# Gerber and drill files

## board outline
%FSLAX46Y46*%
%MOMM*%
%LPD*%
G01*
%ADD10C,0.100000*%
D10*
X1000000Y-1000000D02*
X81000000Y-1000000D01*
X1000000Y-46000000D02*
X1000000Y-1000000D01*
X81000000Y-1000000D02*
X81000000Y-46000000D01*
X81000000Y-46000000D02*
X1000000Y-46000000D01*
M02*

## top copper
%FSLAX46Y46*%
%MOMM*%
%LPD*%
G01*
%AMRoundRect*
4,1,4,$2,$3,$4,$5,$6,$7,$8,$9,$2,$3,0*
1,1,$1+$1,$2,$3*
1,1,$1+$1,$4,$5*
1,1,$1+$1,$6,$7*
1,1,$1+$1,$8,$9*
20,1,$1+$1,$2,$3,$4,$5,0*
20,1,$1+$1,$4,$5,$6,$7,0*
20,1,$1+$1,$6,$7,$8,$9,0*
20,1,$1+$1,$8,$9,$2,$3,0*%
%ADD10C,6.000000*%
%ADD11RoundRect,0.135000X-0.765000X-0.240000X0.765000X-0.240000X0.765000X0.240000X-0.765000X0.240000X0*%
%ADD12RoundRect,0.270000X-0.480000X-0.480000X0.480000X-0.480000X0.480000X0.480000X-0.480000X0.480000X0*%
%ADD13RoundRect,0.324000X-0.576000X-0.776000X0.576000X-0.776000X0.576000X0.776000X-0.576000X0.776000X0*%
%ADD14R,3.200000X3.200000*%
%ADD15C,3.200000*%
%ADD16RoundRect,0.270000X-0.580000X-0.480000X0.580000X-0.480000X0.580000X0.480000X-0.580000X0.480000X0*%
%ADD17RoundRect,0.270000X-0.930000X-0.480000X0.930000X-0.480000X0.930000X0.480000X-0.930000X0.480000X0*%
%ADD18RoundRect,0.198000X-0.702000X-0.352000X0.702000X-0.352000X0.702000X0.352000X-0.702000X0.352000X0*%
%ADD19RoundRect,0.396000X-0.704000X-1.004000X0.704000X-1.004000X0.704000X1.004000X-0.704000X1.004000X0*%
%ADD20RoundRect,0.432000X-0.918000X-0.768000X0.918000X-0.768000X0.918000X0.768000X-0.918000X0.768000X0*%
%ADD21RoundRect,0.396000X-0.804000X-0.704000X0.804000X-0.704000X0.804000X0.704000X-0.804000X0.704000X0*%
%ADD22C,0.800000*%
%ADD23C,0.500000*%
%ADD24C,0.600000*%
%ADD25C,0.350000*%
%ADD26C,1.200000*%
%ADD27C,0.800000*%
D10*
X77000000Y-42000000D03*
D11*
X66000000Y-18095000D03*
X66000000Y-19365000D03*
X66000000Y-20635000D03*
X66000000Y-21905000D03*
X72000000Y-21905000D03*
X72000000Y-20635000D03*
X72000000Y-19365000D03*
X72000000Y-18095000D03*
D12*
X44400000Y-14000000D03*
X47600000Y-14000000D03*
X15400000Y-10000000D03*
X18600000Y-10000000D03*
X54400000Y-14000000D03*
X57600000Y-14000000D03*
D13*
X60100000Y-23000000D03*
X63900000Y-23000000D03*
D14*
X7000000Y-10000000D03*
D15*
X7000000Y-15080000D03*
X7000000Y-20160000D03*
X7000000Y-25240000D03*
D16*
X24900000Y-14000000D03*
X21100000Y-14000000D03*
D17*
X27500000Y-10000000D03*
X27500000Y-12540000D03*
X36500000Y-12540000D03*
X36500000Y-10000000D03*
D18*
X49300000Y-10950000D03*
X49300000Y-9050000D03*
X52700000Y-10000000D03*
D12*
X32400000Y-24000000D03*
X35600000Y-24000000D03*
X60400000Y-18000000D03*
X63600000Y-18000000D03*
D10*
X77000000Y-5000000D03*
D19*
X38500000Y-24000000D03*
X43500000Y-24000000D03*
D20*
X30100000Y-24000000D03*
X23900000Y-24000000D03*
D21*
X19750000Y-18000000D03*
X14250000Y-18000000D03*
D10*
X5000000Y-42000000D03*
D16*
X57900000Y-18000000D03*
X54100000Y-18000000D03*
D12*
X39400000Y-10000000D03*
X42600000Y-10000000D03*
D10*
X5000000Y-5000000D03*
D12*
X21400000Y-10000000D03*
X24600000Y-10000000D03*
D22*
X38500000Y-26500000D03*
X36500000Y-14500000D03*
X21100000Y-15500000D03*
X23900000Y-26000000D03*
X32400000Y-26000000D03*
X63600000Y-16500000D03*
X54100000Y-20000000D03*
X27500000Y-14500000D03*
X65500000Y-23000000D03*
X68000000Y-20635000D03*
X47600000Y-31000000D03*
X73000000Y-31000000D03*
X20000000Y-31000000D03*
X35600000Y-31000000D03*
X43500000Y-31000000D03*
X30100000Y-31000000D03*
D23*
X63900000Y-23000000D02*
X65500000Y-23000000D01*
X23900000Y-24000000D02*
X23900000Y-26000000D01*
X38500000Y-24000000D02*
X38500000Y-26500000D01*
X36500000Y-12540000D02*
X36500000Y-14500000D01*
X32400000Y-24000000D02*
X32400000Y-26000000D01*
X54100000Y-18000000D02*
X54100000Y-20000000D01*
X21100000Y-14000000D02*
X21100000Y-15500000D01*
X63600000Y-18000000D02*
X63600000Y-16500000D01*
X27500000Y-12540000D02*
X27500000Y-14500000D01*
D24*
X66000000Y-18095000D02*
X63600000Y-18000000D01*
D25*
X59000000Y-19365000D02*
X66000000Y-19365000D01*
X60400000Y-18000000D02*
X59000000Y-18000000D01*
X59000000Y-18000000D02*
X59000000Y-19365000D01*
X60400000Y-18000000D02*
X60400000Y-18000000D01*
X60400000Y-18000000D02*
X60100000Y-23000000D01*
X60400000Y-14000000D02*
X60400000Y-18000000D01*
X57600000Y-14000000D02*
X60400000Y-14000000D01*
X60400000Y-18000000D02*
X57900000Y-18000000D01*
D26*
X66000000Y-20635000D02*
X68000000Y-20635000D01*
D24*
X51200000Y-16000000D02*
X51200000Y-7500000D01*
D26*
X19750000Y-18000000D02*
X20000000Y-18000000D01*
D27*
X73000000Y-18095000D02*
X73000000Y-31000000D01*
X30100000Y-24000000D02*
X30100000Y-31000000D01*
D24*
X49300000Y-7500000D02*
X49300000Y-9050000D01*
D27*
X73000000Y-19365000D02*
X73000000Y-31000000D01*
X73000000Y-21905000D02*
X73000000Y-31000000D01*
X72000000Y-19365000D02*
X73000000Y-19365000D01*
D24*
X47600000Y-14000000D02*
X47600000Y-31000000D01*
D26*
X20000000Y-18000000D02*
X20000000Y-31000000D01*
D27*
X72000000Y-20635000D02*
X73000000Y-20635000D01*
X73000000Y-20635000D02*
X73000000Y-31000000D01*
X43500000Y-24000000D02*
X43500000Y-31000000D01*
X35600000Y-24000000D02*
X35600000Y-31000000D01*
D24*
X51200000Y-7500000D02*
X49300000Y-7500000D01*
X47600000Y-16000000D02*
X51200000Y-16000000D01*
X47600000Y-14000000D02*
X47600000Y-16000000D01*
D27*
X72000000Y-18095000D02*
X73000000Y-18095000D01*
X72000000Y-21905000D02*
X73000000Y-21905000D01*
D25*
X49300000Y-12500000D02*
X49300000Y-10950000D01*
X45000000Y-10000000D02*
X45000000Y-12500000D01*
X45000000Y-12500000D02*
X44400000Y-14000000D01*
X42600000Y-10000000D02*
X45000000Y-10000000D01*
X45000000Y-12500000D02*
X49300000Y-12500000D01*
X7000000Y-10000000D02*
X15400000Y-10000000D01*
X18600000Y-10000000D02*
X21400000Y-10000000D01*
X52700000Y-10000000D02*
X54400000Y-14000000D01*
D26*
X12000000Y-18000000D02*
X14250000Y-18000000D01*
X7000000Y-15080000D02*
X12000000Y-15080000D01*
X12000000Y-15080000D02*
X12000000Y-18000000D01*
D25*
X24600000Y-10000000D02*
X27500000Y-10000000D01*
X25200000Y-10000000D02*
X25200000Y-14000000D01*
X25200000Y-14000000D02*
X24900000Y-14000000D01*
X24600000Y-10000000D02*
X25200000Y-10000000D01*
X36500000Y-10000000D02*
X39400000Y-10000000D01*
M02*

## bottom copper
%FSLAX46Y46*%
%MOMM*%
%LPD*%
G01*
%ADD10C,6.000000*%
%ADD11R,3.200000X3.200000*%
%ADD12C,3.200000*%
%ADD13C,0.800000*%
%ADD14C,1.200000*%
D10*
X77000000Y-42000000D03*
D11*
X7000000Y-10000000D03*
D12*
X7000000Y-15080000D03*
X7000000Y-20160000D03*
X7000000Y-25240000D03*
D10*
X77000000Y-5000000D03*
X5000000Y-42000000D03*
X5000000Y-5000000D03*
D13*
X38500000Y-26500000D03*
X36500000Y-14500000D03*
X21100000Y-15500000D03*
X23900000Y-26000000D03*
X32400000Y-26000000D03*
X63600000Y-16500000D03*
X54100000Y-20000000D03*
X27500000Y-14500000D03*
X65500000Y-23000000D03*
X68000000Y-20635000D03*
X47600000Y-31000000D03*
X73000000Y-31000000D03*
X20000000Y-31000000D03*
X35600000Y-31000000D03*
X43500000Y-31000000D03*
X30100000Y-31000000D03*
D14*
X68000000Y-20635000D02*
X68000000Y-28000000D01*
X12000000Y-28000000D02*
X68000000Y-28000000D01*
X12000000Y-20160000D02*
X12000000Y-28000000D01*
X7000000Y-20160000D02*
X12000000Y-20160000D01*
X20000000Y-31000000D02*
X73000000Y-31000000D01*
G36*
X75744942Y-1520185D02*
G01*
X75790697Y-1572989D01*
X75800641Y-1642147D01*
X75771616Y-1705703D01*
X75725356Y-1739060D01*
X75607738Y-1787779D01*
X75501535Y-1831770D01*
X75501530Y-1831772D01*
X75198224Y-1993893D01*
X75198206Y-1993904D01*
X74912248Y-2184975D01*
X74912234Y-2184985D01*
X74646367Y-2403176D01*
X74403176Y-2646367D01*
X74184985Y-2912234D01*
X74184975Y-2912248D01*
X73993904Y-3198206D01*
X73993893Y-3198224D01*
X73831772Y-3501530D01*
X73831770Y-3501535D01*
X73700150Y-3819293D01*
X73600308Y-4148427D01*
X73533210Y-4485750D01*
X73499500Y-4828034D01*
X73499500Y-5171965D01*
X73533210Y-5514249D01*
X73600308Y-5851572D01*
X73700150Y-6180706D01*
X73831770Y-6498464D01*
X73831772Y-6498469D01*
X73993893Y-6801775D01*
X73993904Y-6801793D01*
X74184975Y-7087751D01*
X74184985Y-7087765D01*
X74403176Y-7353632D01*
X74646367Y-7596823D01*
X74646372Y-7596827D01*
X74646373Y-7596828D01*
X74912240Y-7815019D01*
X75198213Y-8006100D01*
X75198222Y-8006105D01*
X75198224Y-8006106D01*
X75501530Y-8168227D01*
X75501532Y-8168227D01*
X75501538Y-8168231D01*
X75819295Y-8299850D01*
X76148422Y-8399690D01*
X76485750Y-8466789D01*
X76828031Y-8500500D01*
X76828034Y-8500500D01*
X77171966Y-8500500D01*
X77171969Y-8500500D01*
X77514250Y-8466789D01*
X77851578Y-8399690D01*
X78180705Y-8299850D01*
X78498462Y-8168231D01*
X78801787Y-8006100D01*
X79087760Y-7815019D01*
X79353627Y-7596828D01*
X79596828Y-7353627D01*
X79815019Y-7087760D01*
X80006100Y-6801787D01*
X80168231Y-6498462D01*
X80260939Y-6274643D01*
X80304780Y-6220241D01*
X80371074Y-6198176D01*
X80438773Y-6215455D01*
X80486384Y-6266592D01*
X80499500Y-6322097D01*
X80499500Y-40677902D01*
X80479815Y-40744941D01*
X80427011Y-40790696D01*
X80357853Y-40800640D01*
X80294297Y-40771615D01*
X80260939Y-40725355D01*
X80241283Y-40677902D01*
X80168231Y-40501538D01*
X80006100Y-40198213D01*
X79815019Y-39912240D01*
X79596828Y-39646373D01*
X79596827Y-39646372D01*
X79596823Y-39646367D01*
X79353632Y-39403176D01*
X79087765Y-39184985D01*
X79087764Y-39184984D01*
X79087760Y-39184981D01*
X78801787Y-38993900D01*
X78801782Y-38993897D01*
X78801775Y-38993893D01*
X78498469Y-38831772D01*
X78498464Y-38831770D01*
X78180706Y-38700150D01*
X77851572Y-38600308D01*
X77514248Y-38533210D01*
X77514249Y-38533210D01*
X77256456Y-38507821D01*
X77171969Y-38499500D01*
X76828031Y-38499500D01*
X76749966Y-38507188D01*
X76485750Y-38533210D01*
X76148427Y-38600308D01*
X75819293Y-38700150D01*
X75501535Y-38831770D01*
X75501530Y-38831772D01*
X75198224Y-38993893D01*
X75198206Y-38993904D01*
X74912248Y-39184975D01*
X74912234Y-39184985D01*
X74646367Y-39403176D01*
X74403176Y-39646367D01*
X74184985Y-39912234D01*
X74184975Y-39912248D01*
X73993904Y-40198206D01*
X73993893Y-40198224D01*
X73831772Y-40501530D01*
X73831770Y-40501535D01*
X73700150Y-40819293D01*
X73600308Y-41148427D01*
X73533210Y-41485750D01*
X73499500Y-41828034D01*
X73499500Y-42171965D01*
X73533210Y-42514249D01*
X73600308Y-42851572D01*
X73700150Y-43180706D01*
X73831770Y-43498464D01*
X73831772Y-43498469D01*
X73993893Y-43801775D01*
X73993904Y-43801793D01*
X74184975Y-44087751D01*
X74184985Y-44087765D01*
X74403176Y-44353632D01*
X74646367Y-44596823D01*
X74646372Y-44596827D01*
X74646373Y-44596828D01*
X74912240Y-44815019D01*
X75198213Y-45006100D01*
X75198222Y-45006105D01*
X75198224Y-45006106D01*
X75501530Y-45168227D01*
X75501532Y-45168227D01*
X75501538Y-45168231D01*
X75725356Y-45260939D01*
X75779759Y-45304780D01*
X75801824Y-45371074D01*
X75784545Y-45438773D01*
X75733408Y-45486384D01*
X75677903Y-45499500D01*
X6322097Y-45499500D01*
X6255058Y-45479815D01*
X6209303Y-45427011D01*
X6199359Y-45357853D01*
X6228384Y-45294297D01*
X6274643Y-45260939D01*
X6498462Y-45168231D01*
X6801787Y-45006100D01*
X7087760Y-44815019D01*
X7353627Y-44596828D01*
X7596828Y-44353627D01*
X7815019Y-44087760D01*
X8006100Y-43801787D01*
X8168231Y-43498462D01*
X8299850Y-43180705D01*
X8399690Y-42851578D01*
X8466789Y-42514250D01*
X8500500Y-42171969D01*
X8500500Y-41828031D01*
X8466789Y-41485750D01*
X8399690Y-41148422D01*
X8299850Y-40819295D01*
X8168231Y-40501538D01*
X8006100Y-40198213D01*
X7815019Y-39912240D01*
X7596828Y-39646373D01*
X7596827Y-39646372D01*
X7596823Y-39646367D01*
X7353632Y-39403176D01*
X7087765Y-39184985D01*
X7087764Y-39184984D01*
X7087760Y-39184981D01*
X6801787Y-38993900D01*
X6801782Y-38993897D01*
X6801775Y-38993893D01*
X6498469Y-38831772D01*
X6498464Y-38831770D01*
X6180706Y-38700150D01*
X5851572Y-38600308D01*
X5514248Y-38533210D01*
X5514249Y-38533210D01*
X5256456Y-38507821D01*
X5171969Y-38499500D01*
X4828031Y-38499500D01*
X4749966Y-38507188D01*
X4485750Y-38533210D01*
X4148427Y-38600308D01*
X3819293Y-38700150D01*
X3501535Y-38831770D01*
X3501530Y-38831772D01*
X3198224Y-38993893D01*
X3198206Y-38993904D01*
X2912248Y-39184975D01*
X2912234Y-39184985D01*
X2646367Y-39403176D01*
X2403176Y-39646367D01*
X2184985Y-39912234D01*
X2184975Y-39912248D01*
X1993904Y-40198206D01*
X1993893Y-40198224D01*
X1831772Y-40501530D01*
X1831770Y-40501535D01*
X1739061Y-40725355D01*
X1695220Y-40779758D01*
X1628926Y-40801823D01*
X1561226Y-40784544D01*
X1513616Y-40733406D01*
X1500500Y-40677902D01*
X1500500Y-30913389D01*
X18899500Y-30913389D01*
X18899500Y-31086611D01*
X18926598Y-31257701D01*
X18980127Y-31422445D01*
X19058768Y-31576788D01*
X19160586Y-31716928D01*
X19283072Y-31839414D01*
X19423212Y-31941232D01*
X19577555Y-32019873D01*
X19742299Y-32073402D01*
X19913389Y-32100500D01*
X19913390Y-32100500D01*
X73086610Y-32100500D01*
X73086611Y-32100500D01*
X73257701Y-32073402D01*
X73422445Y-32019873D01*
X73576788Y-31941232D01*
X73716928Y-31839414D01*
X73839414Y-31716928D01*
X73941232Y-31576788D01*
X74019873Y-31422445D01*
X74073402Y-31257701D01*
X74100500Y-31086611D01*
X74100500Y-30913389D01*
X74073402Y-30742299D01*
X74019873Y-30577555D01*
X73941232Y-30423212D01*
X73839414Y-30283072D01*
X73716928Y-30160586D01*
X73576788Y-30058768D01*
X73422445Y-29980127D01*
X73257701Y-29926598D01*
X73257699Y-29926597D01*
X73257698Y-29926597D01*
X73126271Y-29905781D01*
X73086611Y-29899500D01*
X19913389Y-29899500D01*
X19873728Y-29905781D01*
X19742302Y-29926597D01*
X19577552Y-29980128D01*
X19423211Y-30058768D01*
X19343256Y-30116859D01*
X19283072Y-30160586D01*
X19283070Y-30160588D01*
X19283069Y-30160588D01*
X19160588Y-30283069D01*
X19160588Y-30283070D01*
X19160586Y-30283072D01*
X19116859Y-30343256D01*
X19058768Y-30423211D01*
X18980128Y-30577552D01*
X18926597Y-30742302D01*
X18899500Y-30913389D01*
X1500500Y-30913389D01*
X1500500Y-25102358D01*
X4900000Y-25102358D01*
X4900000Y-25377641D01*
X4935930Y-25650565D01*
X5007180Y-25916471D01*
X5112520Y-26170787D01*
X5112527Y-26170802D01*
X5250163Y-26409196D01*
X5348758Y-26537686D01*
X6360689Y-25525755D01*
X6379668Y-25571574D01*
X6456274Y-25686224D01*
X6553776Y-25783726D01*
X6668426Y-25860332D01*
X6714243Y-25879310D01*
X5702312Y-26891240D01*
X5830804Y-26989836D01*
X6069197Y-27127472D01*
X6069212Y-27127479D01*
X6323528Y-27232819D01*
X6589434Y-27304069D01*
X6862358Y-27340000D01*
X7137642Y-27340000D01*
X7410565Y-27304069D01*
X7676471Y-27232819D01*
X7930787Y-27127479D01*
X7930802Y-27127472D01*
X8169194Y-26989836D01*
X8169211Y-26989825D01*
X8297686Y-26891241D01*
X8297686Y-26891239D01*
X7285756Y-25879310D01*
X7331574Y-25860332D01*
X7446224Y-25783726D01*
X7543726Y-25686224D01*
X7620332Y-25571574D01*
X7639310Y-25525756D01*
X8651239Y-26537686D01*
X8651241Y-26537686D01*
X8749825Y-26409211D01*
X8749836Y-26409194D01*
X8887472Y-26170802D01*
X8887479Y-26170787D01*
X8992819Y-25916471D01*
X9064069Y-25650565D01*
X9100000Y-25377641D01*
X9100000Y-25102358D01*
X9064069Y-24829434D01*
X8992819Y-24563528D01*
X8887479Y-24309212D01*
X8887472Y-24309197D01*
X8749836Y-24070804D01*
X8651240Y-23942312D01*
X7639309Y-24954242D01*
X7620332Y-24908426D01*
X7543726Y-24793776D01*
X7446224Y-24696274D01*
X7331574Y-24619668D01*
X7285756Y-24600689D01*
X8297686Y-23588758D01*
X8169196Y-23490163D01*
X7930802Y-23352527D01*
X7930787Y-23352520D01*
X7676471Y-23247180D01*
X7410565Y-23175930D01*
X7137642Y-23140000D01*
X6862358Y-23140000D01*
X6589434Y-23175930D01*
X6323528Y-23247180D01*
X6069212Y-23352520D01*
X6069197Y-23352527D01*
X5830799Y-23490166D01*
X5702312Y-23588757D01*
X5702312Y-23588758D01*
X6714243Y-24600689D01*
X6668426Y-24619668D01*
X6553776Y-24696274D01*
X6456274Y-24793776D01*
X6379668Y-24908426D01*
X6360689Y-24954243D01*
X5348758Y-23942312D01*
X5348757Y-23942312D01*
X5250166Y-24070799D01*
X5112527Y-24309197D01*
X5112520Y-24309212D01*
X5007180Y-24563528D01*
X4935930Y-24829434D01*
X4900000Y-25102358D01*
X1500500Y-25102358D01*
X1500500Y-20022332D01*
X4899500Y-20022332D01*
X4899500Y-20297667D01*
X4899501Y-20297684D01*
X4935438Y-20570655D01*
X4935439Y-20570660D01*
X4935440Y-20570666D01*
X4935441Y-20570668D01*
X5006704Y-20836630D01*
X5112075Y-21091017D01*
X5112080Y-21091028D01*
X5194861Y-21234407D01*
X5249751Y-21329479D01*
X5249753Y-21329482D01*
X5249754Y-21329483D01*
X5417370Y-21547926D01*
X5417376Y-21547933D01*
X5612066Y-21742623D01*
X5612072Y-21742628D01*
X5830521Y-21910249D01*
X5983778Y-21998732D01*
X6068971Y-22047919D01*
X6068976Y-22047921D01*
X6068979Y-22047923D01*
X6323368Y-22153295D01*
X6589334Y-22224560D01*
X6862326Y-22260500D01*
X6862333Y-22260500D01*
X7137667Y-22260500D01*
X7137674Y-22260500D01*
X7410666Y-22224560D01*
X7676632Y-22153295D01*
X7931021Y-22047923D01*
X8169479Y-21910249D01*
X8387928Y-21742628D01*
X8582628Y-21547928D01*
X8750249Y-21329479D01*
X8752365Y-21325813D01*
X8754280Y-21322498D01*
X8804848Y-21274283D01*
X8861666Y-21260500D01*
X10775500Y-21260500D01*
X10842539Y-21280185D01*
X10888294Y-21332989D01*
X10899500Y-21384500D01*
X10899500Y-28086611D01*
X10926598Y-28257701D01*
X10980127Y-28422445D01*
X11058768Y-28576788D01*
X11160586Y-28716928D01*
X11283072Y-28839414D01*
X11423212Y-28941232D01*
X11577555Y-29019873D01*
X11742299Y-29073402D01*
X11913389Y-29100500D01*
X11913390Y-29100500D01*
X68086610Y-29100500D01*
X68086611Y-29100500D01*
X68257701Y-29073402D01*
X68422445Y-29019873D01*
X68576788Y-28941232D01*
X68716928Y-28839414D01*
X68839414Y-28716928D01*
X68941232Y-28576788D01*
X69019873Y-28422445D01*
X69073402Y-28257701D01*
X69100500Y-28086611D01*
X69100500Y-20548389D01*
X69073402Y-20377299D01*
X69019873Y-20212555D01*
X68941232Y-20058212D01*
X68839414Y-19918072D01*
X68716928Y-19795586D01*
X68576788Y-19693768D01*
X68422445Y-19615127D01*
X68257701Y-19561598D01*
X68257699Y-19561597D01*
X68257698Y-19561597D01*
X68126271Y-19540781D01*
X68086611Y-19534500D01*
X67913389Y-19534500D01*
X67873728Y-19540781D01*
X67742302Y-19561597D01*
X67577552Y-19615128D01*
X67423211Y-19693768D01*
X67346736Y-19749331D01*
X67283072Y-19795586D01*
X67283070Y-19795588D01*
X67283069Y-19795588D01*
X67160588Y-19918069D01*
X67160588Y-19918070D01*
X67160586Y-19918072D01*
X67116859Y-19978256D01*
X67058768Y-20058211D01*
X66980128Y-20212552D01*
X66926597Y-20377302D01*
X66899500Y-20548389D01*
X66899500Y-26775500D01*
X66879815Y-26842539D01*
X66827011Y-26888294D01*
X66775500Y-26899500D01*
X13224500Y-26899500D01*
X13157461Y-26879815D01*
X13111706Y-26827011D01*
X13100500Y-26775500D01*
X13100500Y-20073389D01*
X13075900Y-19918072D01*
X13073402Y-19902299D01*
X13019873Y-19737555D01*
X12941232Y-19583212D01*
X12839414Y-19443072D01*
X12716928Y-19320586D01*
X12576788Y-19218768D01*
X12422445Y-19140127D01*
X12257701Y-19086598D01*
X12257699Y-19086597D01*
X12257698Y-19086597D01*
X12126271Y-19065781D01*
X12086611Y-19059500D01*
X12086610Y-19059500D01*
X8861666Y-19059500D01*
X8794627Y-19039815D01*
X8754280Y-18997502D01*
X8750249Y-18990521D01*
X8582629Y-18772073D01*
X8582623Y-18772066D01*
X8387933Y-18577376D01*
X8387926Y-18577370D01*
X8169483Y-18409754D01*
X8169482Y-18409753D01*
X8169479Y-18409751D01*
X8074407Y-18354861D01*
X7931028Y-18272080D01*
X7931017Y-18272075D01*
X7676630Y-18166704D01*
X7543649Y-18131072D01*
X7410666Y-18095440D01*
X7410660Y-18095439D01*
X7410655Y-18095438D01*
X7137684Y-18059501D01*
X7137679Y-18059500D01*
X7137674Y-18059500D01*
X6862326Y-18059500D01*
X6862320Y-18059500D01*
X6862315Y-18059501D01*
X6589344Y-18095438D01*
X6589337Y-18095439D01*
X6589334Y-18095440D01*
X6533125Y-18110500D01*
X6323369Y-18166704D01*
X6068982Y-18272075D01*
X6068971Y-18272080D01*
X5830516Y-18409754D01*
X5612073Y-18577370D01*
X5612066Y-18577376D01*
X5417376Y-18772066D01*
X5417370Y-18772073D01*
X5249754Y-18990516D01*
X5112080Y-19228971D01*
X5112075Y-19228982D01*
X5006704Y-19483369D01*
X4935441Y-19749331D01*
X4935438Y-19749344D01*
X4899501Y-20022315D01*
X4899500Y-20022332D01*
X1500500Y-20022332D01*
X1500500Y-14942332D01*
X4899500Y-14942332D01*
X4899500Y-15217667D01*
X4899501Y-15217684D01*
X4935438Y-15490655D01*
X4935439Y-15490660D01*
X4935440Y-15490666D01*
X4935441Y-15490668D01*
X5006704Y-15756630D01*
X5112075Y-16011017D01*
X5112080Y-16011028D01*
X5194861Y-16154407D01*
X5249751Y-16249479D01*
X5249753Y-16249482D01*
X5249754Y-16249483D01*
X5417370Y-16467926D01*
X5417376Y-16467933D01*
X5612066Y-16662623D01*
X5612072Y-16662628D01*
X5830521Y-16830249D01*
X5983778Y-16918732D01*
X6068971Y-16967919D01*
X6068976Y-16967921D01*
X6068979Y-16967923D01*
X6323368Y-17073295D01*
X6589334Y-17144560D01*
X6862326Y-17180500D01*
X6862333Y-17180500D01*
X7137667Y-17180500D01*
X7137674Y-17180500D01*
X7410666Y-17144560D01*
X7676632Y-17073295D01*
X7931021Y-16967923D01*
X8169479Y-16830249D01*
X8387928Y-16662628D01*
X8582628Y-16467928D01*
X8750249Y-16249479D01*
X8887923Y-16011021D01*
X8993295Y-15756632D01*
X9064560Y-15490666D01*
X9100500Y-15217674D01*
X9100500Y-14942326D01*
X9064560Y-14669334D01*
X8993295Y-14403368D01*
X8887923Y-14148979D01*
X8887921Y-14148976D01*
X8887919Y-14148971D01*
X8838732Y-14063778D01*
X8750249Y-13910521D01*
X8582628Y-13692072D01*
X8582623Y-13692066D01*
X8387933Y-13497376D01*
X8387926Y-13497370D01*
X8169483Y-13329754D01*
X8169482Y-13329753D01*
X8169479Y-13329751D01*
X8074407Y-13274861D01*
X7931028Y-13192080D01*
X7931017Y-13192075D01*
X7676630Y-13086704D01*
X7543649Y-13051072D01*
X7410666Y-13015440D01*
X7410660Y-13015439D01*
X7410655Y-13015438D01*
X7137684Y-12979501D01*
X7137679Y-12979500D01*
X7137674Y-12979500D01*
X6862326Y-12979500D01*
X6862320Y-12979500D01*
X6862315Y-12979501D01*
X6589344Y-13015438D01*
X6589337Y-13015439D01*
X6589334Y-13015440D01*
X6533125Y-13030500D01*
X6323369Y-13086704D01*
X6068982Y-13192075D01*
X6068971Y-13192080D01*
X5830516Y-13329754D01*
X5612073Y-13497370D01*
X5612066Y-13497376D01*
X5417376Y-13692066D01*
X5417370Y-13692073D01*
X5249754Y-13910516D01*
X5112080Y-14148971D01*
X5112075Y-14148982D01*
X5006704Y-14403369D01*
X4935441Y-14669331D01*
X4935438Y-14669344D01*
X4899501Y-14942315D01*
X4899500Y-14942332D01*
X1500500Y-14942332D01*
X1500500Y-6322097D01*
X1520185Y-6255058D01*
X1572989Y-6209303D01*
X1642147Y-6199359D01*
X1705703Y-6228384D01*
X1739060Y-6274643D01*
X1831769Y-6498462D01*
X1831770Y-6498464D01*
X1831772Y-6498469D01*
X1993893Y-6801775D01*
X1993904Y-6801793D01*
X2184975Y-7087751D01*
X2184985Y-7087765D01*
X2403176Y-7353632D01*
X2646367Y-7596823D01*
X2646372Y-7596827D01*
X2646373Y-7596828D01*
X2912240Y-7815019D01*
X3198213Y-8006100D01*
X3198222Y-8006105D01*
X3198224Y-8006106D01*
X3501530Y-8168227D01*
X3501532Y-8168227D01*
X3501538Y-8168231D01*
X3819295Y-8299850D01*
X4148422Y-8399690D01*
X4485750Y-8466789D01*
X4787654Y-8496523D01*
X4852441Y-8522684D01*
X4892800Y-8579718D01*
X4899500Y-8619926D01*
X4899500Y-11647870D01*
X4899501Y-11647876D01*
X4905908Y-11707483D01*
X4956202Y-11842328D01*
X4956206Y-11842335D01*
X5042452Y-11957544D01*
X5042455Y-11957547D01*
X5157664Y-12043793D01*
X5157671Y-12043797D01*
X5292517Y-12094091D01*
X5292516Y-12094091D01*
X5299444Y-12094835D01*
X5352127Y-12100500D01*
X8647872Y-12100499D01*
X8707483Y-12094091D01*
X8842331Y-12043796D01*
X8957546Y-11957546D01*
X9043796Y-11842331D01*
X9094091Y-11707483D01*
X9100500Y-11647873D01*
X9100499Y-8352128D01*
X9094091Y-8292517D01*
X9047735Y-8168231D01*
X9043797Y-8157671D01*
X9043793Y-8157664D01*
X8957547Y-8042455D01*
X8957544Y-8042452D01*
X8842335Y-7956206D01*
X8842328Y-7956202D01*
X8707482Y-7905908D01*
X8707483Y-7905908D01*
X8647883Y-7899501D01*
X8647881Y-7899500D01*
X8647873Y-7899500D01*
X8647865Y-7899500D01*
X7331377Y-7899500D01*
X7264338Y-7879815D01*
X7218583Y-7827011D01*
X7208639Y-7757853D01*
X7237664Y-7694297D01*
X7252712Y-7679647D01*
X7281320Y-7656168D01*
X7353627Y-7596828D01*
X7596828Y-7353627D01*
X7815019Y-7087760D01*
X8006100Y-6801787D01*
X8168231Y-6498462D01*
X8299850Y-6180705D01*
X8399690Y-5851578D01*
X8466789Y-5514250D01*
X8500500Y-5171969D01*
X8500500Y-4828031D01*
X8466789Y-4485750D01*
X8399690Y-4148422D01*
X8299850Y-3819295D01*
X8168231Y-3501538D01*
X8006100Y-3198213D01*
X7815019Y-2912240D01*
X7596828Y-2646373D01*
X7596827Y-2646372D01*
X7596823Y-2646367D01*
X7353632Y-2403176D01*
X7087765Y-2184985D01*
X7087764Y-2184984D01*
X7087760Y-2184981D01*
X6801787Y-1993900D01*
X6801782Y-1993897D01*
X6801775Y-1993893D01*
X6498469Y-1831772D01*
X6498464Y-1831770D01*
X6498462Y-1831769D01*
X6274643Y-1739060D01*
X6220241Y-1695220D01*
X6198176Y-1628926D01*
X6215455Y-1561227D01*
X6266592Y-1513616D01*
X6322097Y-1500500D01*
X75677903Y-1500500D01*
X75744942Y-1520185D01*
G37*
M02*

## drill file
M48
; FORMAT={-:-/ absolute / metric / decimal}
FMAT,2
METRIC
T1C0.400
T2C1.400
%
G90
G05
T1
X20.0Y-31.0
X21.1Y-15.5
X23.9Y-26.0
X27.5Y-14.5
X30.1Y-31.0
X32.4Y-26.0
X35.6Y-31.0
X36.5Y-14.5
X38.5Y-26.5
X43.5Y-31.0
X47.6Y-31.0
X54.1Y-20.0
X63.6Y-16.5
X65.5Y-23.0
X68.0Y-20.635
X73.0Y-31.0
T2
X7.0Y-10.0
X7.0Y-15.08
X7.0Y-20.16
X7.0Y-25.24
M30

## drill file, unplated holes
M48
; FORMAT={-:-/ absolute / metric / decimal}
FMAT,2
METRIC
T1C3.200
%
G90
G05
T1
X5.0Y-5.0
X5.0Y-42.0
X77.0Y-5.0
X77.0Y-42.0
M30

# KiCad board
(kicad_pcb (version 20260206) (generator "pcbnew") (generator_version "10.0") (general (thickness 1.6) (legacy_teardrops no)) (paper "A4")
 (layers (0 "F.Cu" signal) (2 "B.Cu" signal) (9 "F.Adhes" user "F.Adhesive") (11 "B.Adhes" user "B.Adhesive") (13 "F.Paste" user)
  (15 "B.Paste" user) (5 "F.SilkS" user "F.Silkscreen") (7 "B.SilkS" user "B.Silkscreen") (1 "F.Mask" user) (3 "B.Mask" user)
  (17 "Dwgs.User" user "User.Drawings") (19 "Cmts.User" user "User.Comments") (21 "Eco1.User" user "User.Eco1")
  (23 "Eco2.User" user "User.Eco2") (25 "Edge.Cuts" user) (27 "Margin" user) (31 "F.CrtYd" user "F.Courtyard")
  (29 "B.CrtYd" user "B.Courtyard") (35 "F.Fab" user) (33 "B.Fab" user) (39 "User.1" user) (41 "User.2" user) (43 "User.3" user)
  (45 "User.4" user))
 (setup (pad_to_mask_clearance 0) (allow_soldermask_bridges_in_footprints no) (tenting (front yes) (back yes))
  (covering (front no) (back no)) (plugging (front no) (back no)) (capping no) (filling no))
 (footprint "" (layer "F.Cu") (at 0 0)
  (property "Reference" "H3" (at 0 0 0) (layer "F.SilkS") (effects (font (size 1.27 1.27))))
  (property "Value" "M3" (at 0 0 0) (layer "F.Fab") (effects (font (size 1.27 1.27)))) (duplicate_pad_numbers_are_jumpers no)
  (pad "" np_thru_hole circle (at 77 42) (size 6 6) (drill 3.2) (layers "*.Cu" "*.Mask")))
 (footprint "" (layer "F.Cu") (at 0 0)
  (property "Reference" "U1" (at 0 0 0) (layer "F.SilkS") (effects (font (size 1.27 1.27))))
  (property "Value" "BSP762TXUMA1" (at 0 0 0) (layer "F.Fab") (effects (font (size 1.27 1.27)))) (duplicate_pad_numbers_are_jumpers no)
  (pad "1" smd roundrect (at 66 18.095) (size 1.8 0.75) (layers "F.Cu" "F.Mask" "F.Paste") (roundrect_rratio 0.18) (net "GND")
   (thermal_bridge_angle 45))
  (pad "2" smd roundrect (at 66 19.365) (size 1.8 0.75) (layers "F.Cu" "F.Mask" "F.Paste") (roundrect_rratio 0.18) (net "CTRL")
   (thermal_bridge_angle 45))
  (pad "3" smd roundrect (at 66 20.635) (size 1.8 0.75) (layers "F.Cu" "F.Mask" "F.Paste") (roundrect_rratio 0.18) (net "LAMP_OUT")
   (thermal_bridge_angle 45))
  (pad "4" smd roundrect (at 66 21.905) (size 1.8 0.75) (layers "F.Cu" "F.Mask" "F.Paste") (roundrect_rratio 0.18) (thermal_bridge_angle 45))
  (pad "5" smd roundrect (at 72 21.905) (size 1.8 0.75) (layers "F.Cu" "F.Mask" "F.Paste") (roundrect_rratio 0.18) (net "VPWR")
   (thermal_bridge_angle 45))
  (pad "6" smd roundrect (at 72 20.635) (size 1.8 0.75) (layers "F.Cu" "F.Mask" "F.Paste") (roundrect_rratio 0.18) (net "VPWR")
   (thermal_bridge_angle 45))
  (pad "7" smd roundrect (at 72 19.365) (size 1.8 0.75) (layers "F.Cu" "F.Mask" "F.Paste") (roundrect_rratio 0.18) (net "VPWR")
   (thermal_bridge_angle 45))
  (pad "8" smd roundrect (at 72 18.095) (size 1.8 0.75) (layers "F.Cu" "F.Mask" "F.Paste") (roundrect_rratio 0.18) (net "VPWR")
   (thermal_bridge_angle 45)))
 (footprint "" (layer "F.Cu") (at 0 0)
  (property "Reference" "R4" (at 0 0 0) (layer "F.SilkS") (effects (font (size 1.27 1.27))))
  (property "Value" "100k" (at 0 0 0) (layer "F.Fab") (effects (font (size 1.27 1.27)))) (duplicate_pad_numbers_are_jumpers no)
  (pad "1" smd roundrect (at 44.4 14) (size 1.5 1.5) (layers "F.Cu" "F.Mask" "F.Paste") (roundrect_rratio 0.18) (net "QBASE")
   (thermal_bridge_angle 45))
  (pad "2" smd roundrect (at 47.6 14) (size 1.5 1.5) (layers "F.Cu" "F.Mask" "F.Paste") (roundrect_rratio 0.18) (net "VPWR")
   (thermal_bridge_angle 45)))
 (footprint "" (layer "F.Cu") (at 0 0)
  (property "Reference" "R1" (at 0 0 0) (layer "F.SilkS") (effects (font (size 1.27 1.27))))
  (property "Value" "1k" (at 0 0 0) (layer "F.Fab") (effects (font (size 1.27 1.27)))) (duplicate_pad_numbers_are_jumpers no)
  (pad "1" smd roundrect (at 15.4 10) (size 1.5 1.5) (layers "F.Cu" "F.Mask" "F.Paste") (roundrect_rratio 0.18) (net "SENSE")
   (thermal_bridge_angle 45))
  (pad "2" smd roundrect (at 18.6 10) (size 1.5 1.5) (layers "F.Cu" "F.Mask" "F.Paste") (roundrect_rratio 0.18) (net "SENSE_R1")
   (thermal_bridge_angle 45)))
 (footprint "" (layer "F.Cu") (at 0 0)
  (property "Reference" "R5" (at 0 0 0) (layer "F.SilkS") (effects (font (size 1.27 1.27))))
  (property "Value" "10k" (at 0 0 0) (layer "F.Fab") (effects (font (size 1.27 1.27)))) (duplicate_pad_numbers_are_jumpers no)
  (pad "1" smd roundrect (at 54.4 14) (size 1.5 1.5) (layers "F.Cu" "F.Mask" "F.Paste") (roundrect_rratio 0.18) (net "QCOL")
   (thermal_bridge_angle 45))
  (pad "2" smd roundrect (at 57.6 14) (size 1.5 1.5) (layers "F.Cu" "F.Mask" "F.Paste") (roundrect_rratio 0.18) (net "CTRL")
   (thermal_bridge_angle 45)))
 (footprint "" (layer "F.Cu") (at 0 0)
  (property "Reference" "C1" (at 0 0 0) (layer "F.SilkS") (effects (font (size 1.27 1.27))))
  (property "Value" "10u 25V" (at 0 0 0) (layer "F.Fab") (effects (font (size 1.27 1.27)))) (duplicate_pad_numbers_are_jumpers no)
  (pad "1" smd roundrect (at 60.1 23) (size 1.8 2.2) (layers "F.Cu" "F.Mask" "F.Paste") (roundrect_rratio 0.18) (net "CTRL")
   (thermal_bridge_angle 45))
  (pad "2" smd roundrect (at 63.9 23) (size 1.8 2.2) (layers "F.Cu" "F.Mask" "F.Paste") (roundrect_rratio 0.18) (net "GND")
   (thermal_bridge_angle 45)))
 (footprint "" (layer "F.Cu") (at 0 0)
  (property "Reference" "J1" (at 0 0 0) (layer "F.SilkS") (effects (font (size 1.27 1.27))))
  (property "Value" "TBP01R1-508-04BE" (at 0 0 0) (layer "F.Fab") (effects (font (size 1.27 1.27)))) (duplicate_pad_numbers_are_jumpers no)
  (pad "1" thru_hole rect (at 7 10) (size 3.2 3.2) (drill 1.4) (layers "*.Cu" "*.Mask") (remove_unused_layers no) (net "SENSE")
   (thermal_bridge_angle 45))
  (pad "2" thru_hole circle (at 7 15.08) (size 3.2 3.2) (drill 1.4) (layers "*.Cu" "*.Mask") (remove_unused_layers no) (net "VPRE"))
  (pad "3" thru_hole circle (at 7 20.16) (size 3.2 3.2) (drill 1.4) (layers "*.Cu" "*.Mask") (remove_unused_layers no) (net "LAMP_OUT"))
  (pad "4" thru_hole circle (at 7 25.24) (size 3.2 3.2) (drill 1.4) (layers "*.Cu" "*.Mask") (remove_unused_layers no) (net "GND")))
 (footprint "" (layer "F.Cu") (at 0 0)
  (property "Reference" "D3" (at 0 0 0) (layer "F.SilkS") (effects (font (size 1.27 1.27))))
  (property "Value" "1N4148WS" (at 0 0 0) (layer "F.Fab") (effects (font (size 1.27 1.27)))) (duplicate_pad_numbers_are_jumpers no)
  (pad "1" smd roundrect (at 24.9 14) (size 1.7 1.5) (layers "F.Cu" "F.Mask" "F.Paste") (roundrect_rratio 0.18) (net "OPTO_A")
   (thermal_bridge_angle 45))
  (pad "2" smd roundrect (at 21.1 14) (size 1.7 1.5) (layers "F.Cu" "F.Mask" "F.Paste") (roundrect_rratio 0.18) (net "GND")
   (thermal_bridge_angle 45)))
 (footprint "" (layer "F.Cu") (at 0 0)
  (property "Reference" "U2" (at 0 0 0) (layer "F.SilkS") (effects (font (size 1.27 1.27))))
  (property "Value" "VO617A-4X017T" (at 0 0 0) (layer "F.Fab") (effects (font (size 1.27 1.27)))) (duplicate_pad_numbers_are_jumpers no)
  (pad "1" smd roundrect (at 27.5 10) (size 2.4 1.5) (layers "F.Cu" "F.Mask" "F.Paste") (roundrect_rratio 0.18) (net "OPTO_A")
   (thermal_bridge_angle 45))
  (pad "2" smd roundrect (at 27.5 12.54) (size 2.4 1.5) (layers "F.Cu" "F.Mask" "F.Paste") (roundrect_rratio 0.18) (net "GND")
   (thermal_bridge_angle 45))
  (pad "3" smd roundrect (at 36.5 12.54) (size 2.4 1.5) (layers "F.Cu" "F.Mask" "F.Paste") (roundrect_rratio 0.18) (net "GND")
   (thermal_bridge_angle 45))
  (pad "4" smd roundrect (at 36.5 10) (size 2.4 1.5) (layers "F.Cu" "F.Mask" "F.Paste") (roundrect_rratio 0.18) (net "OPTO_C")
   (thermal_bridge_angle 45)))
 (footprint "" (layer "F.Cu") (at 0 0)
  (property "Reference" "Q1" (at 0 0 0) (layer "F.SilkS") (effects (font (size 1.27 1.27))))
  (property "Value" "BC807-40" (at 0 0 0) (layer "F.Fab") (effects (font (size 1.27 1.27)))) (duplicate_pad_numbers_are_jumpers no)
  (pad "1" smd roundrect (at 49.3 10.95) (size 1.8 1.1) (layers "F.Cu" "F.Mask" "F.Paste") (roundrect_rratio 0.18) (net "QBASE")
   (thermal_bridge_angle 45))
  (pad "2" smd roundrect (at 49.3 9.05) (size 1.8 1.1) (layers "F.Cu" "F.Mask" "F.Paste") (roundrect_rratio 0.18) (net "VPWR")
   (thermal_bridge_angle 45))
  (pad "3" smd roundrect (at 52.7 10) (size 1.8 1.1) (layers "F.Cu" "F.Mask" "F.Paste") (roundrect_rratio 0.18) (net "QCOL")
   (thermal_bridge_angle 45)))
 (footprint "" (layer "F.Cu") (at 0 0)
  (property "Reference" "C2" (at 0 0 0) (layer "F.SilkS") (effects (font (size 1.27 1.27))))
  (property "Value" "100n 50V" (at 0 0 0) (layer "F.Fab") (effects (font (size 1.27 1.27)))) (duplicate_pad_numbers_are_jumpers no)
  (pad "1" smd roundrect (at 32.4 24) (size 1.5 1.5) (layers "F.Cu" "F.Mask" "F.Paste") (roundrect_rratio 0.18) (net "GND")
   (thermal_bridge_angle 45))
  (pad "2" smd roundrect (at 35.6 24) (size 1.5 1.5) (layers "F.Cu" "F.Mask" "F.Paste") (roundrect_rratio 0.18) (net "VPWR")
   (thermal_bridge_angle 45)))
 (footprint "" (layer "F.Cu") (at 0 0)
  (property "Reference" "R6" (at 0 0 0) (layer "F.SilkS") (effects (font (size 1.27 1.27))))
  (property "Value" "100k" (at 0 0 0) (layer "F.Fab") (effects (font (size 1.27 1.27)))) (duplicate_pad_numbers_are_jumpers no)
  (pad "1" smd roundrect (at 60.4 18) (size 1.5 1.5) (layers "F.Cu" "F.Mask" "F.Paste") (roundrect_rratio 0.18) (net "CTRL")
   (thermal_bridge_angle 45))
  (pad "2" smd roundrect (at 63.6 18) (size 1.5 1.5) (layers "F.Cu" "F.Mask" "F.Paste") (roundrect_rratio 0.18) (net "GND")
   (thermal_bridge_angle 45)))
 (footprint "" (layer "F.Cu") (at 0 0)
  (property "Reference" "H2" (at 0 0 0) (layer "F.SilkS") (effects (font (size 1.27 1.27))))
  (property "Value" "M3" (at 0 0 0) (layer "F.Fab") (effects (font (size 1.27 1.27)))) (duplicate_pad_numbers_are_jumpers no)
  (pad "" np_thru_hole circle (at 77 5) (size 6 6) (drill 3.2) (layers "*.Cu" "*.Mask")))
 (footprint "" (layer "F.Cu") (at 0 0)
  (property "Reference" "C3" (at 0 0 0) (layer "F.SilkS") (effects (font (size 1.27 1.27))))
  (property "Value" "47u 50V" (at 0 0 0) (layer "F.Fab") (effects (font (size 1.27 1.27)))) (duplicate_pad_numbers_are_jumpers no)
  (pad "1" smd roundrect (at 38.5 24) (size 2.2 2.8) (layers "F.Cu" "F.Mask" "F.Paste") (roundrect_rratio 0.18) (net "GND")
   (thermal_bridge_angle 45))
  (pad "2" smd roundrect (at 43.5 24) (size 2.2 2.8) (layers "F.Cu" "F.Mask" "F.Paste") (roundrect_rratio 0.18) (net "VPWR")
   (thermal_bridge_angle 45)))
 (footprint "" (layer "F.Cu") (at 0 0)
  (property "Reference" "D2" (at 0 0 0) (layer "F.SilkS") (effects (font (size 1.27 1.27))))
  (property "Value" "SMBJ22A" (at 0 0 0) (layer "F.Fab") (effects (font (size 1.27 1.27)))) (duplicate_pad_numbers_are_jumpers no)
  (pad "1" smd roundrect (at 30.1 24) (size 2.7 2.4) (layers "F.Cu" "F.Mask" "F.Paste") (roundrect_rratio 0.18) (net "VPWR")
   (thermal_bridge_angle 45))
  (pad "2" smd roundrect (at 23.9 24) (size 2.7 2.4) (layers "F.Cu" "F.Mask" "F.Paste") (roundrect_rratio 0.18) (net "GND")
   (thermal_bridge_angle 45)))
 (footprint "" (layer "F.Cu") (at 0 0)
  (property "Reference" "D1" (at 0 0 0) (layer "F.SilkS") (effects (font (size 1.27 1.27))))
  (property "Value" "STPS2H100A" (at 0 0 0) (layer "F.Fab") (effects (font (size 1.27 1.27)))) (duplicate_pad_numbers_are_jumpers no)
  (pad "1" smd roundrect (at 19.75 18) (size 2.4 2.2) (layers "F.Cu" "F.Mask" "F.Paste") (roundrect_rratio 0.18) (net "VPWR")
   (thermal_bridge_angle 45))
  (pad "2" smd roundrect (at 14.25 18) (size 2.4 2.2) (layers "F.Cu" "F.Mask" "F.Paste") (roundrect_rratio 0.18) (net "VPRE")
   (thermal_bridge_angle 45)))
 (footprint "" (layer "F.Cu") (at 0 0)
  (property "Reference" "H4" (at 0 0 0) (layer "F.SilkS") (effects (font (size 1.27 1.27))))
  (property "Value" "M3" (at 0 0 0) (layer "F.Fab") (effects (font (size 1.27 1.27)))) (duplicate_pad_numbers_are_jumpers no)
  (pad "" np_thru_hole circle (at 5 42) (size 6 6) (drill 3.2) (layers "*.Cu" "*.Mask")))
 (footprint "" (layer "F.Cu") (at 0 0)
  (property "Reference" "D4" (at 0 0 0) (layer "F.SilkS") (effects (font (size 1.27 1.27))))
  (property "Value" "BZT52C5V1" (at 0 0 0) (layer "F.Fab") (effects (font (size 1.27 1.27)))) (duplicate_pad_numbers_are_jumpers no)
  (pad "1" smd roundrect (at 57.9 18) (size 1.7 1.5) (layers "F.Cu" "F.Mask" "F.Paste") (roundrect_rratio 0.18) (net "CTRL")
   (thermal_bridge_angle 45))
  (pad "2" smd roundrect (at 54.1 18) (size 1.7 1.5) (layers "F.Cu" "F.Mask" "F.Paste") (roundrect_rratio 0.18) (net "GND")
   (thermal_bridge_angle 45)))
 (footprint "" (layer "F.Cu") (at 0 0)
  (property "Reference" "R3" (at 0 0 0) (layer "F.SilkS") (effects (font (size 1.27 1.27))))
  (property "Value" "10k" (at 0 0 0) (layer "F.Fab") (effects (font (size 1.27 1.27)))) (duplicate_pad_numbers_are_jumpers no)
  (pad "1" smd roundrect (at 39.4 10) (size 1.5 1.5) (layers "F.Cu" "F.Mask" "F.Paste") (roundrect_rratio 0.18) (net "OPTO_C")
   (thermal_bridge_angle 45))
  (pad "2" smd roundrect (at 42.6 10) (size 1.5 1.5) (layers "F.Cu" "F.Mask" "F.Paste") (roundrect_rratio 0.18) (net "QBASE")
   (thermal_bridge_angle 45)))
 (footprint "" (layer "F.Cu") (at 0 0)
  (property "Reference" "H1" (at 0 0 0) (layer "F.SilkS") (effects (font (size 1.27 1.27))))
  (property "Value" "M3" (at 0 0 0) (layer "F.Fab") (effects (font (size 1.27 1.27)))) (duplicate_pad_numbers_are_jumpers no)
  (pad "" np_thru_hole circle (at 5 5) (size 6 6) (drill 3.2) (layers "*.Cu" "*.Mask")))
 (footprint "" (layer "F.Cu") (at 0 0)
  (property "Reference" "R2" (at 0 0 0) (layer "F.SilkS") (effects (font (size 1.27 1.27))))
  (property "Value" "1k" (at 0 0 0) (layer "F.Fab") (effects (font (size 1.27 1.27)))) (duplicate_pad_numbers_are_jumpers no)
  (pad "1" smd roundrect (at 21.4 10) (size 1.5 1.5) (layers "F.Cu" "F.Mask" "F.Paste") (roundrect_rratio 0.18) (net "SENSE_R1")
   (thermal_bridge_angle 45))
  (pad "2" smd roundrect (at 24.6 10) (size 1.5 1.5) (layers "F.Cu" "F.Mask" "F.Paste") (roundrect_rratio 0.18) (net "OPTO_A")
   (thermal_bridge_angle 45)))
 (gr_line (start 1 1) (end 81 1) (stroke (width 0.1) (type default)) (layer "Edge.Cuts"))
 (gr_line (start 1 46) (end 1 1) (stroke (width 0.1) (type default)) (layer "Edge.Cuts"))
 (gr_line (start 81 1) (end 81 46) (stroke (width 0.1) (type default)) (layer "Edge.Cuts"))
 (gr_line (start 81 46) (end 1 46) (stroke (width 0.1) (type default)) (layer "Edge.Cuts"))
 (segment (start 63.9 23) (end 65.5 23) (width 0.5) (layer "F.Cu") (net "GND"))
 (segment (start 23.9 24) (end 23.9 26) (width 0.5) (layer "F.Cu") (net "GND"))
 (segment (start 38.5 24) (end 38.5 26.5) (width 0.5) (layer "F.Cu") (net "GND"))
 (segment (start 36.5 12.54) (end 36.5 14.5) (width 0.5) (layer "F.Cu") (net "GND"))
 (segment (start 32.4 24) (end 32.4 26) (width 0.5) (layer "F.Cu") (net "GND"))
 (segment (start 54.1 18) (end 54.1 20) (width 0.5) (layer "F.Cu") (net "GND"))
 (segment (start 21.1 14) (end 21.1 15.5) (width 0.5) (layer "F.Cu") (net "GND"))
 (segment (start 63.6 18) (end 63.6 16.5) (width 0.5) (layer "F.Cu") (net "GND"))
 (segment (start 27.5 12.54) (end 27.5 14.5) (width 0.5) (layer "F.Cu") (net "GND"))
 (segment (start 66 18.095) (end 63.6 18) (width 0.6) (layer "F.Cu") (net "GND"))
 (via (at 38.5 26.5) (size 0.8) (drill 0.4) (layers "F.Cu" "B.Cu") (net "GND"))
 (via (at 36.5 14.5) (size 0.8) (drill 0.4) (layers "F.Cu" "B.Cu") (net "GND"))
 (via (at 21.1 15.5) (size 0.8) (drill 0.4) (layers "F.Cu" "B.Cu") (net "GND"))
 (via (at 23.9 26) (size 0.8) (drill 0.4) (layers "F.Cu" "B.Cu") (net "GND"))
 (via (at 32.4 26) (size 0.8) (drill 0.4) (layers "F.Cu" "B.Cu") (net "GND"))
 (via (at 63.6 16.5) (size 0.8) (drill 0.4) (layers "F.Cu" "B.Cu") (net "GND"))
 (via (at 54.1 20) (size 0.8) (drill 0.4) (layers "F.Cu" "B.Cu") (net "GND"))
 (via (at 27.5 14.5) (size 0.8) (drill 0.4) (layers "F.Cu" "B.Cu") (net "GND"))
 (via (at 65.5 23) (size 0.8) (drill 0.4) (layers "F.Cu" "B.Cu") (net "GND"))
 (segment (start 59 19.365) (end 66 19.365) (width 0.35) (layer "F.Cu") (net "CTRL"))
 (segment (start 60.4 18) (end 59 18) (width 0.35) (layer "F.Cu") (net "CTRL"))
 (segment (start 59 18) (end 59 19.365) (width 0.35) (layer "F.Cu") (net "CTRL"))
 (segment (start 60.4 18) (end 60.4 18) (width 0.35) (layer "F.Cu") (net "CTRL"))
 (segment (start 60.4 18) (end 60.1 23) (width 0.35) (layer "F.Cu") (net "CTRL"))
 (segment (start 60.4 14) (end 60.4 18) (width 0.35) (layer "F.Cu") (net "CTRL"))
 (segment (start 57.6 14) (end 60.4 14) (width 0.35) (layer "F.Cu") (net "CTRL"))
 (segment (start 60.4 18) (end 57.9 18) (width 0.35) (layer "F.Cu") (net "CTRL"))
 (segment (start 66 20.635) (end 68 20.635) (width 1.2) (layer "F.Cu") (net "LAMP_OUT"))
 (via (at 68 20.635) (size 0.8) (drill 0.4) (layers "F.Cu" "B.Cu") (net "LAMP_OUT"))
 (segment (start 68 20.635) (end 68 28) (width 1.2) (layer "B.Cu") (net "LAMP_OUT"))
 (segment (start 12 28) (end 68 28) (width 1.2) (layer "B.Cu") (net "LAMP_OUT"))
 (segment (start 12 20.16) (end 12 28) (width 1.2) (layer "B.Cu") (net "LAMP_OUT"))
 (segment (start 7 20.16) (end 12 20.16) (width 1.2) (layer "B.Cu") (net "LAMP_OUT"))
 (segment (start 51.2 16) (end 51.2 7.5) (width 0.6) (layer "F.Cu") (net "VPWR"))
 (segment (start 19.75 18) (end 20 18) (width 1.2) (layer "F.Cu") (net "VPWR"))
 (segment (start 73 18.095) (end 73 31) (width 0.8) (layer "F.Cu") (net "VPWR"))
 (segment (start 30.1 24) (end 30.1 31) (width 0.8) (layer "F.Cu") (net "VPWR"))
 (segment (start 49.3 7.5) (end 49.3 9.05) (width 0.6) (layer "F.Cu") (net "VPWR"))
 (segment (start 73 19.365) (end 73 31) (width 0.8) (layer "F.Cu") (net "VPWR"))
 (segment (start 73 21.905) (end 73 31) (width 0.8) (layer "F.Cu") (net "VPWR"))
 (segment (start 72 19.365) (end 73 19.365) (width 0.8) (layer "F.Cu") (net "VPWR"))
 (segment (start 47.6 14) (end 47.6 31) (width 0.6) (layer "F.Cu") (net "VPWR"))
 (segment (start 20 18) (end 20 31) (width 1.2) (layer "F.Cu") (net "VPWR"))
 (segment (start 72 20.635) (end 73 20.635) (width 0.8) (layer "F.Cu") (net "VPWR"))
 (segment (start 73 20.635) (end 73 31) (width 0.8) (layer "F.Cu") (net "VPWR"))
 (segment (start 43.5 24) (end 43.5 31) (width 0.8) (layer "F.Cu") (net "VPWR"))
 (segment (start 35.6 24) (end 35.6 31) (width 0.8) (layer "F.Cu") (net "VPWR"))
 (segment (start 51.2 7.5) (end 49.3 7.5) (width 0.6) (layer "F.Cu") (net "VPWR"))
 (segment (start 47.6 16) (end 51.2 16) (width 0.6) (layer "F.Cu") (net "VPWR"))
 (segment (start 47.6 14) (end 47.6 16) (width 0.6) (layer "F.Cu") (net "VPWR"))
 (segment (start 72 18.095) (end 73 18.095) (width 0.8) (layer "F.Cu") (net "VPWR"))
 (segment (start 72 21.905) (end 73 21.905) (width 0.8) (layer "F.Cu") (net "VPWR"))
 (via (at 47.6 31) (size 0.8) (drill 0.4) (layers "F.Cu" "B.Cu") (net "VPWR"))
 (via (at 73 31) (size 0.8) (drill 0.4) (layers "F.Cu" "B.Cu") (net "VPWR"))
 (via (at 20 31) (size 0.8) (drill 0.4) (layers "F.Cu" "B.Cu") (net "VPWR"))
 (via (at 35.6 31) (size 0.8) (drill 0.4) (layers "F.Cu" "B.Cu") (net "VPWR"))
 (via (at 43.5 31) (size 0.8) (drill 0.4) (layers "F.Cu" "B.Cu") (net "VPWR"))
 (via (at 30.1 31) (size 0.8) (drill 0.4) (layers "F.Cu" "B.Cu") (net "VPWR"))
 (segment (start 20 31) (end 73 31) (width 1.2) (layer "B.Cu") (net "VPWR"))
 (segment (start 49.3 12.5) (end 49.3 10.95) (width 0.35) (layer "F.Cu") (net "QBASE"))
 (segment (start 45 10) (end 45 12.5) (width 0.35) (layer "F.Cu") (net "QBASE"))
 (segment (start 45 12.5) (end 44.4 14) (width 0.35) (layer "F.Cu") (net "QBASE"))
 (segment (start 42.6 10) (end 45 10) (width 0.35) (layer "F.Cu") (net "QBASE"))
 (segment (start 45 12.5) (end 49.3 12.5) (width 0.35) (layer "F.Cu") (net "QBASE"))
 (segment (start 7 10) (end 15.4 10) (width 0.35) (layer "F.Cu") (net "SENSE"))
 (segment (start 18.6 10) (end 21.4 10) (width 0.35) (layer "F.Cu") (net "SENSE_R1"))
 (segment (start 52.7 10) (end 54.4 14) (width 0.35) (layer "F.Cu") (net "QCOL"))
 (segment (start 12 18) (end 14.25 18) (width 1.2) (layer "F.Cu") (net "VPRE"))
 (segment (start 7 15.08) (end 12 15.08) (width 1.2) (layer "F.Cu") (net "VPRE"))
 (segment (start 12 15.08) (end 12 18) (width 1.2) (layer "F.Cu") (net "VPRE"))
 (segment (start 24.6 10) (end 27.5 10) (width 0.35) (layer "F.Cu") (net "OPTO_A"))
 (segment (start 25.2 10) (end 25.2 14) (width 0.35) (layer "F.Cu") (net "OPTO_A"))
 (segment (start 25.2 14) (end 24.9 14) (width 0.35) (layer "F.Cu") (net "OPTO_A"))
 (segment (start 24.6 10) (end 25.2 10) (width 0.35) (layer "F.Cu") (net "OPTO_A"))
 (segment (start 36.5 10) (end 39.4 10) (width 0.35) (layer "F.Cu") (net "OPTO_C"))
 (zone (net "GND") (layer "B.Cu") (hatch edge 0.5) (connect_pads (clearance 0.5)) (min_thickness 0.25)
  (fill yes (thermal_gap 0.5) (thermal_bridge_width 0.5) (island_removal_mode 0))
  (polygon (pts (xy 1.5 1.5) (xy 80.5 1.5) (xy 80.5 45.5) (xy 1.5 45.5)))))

